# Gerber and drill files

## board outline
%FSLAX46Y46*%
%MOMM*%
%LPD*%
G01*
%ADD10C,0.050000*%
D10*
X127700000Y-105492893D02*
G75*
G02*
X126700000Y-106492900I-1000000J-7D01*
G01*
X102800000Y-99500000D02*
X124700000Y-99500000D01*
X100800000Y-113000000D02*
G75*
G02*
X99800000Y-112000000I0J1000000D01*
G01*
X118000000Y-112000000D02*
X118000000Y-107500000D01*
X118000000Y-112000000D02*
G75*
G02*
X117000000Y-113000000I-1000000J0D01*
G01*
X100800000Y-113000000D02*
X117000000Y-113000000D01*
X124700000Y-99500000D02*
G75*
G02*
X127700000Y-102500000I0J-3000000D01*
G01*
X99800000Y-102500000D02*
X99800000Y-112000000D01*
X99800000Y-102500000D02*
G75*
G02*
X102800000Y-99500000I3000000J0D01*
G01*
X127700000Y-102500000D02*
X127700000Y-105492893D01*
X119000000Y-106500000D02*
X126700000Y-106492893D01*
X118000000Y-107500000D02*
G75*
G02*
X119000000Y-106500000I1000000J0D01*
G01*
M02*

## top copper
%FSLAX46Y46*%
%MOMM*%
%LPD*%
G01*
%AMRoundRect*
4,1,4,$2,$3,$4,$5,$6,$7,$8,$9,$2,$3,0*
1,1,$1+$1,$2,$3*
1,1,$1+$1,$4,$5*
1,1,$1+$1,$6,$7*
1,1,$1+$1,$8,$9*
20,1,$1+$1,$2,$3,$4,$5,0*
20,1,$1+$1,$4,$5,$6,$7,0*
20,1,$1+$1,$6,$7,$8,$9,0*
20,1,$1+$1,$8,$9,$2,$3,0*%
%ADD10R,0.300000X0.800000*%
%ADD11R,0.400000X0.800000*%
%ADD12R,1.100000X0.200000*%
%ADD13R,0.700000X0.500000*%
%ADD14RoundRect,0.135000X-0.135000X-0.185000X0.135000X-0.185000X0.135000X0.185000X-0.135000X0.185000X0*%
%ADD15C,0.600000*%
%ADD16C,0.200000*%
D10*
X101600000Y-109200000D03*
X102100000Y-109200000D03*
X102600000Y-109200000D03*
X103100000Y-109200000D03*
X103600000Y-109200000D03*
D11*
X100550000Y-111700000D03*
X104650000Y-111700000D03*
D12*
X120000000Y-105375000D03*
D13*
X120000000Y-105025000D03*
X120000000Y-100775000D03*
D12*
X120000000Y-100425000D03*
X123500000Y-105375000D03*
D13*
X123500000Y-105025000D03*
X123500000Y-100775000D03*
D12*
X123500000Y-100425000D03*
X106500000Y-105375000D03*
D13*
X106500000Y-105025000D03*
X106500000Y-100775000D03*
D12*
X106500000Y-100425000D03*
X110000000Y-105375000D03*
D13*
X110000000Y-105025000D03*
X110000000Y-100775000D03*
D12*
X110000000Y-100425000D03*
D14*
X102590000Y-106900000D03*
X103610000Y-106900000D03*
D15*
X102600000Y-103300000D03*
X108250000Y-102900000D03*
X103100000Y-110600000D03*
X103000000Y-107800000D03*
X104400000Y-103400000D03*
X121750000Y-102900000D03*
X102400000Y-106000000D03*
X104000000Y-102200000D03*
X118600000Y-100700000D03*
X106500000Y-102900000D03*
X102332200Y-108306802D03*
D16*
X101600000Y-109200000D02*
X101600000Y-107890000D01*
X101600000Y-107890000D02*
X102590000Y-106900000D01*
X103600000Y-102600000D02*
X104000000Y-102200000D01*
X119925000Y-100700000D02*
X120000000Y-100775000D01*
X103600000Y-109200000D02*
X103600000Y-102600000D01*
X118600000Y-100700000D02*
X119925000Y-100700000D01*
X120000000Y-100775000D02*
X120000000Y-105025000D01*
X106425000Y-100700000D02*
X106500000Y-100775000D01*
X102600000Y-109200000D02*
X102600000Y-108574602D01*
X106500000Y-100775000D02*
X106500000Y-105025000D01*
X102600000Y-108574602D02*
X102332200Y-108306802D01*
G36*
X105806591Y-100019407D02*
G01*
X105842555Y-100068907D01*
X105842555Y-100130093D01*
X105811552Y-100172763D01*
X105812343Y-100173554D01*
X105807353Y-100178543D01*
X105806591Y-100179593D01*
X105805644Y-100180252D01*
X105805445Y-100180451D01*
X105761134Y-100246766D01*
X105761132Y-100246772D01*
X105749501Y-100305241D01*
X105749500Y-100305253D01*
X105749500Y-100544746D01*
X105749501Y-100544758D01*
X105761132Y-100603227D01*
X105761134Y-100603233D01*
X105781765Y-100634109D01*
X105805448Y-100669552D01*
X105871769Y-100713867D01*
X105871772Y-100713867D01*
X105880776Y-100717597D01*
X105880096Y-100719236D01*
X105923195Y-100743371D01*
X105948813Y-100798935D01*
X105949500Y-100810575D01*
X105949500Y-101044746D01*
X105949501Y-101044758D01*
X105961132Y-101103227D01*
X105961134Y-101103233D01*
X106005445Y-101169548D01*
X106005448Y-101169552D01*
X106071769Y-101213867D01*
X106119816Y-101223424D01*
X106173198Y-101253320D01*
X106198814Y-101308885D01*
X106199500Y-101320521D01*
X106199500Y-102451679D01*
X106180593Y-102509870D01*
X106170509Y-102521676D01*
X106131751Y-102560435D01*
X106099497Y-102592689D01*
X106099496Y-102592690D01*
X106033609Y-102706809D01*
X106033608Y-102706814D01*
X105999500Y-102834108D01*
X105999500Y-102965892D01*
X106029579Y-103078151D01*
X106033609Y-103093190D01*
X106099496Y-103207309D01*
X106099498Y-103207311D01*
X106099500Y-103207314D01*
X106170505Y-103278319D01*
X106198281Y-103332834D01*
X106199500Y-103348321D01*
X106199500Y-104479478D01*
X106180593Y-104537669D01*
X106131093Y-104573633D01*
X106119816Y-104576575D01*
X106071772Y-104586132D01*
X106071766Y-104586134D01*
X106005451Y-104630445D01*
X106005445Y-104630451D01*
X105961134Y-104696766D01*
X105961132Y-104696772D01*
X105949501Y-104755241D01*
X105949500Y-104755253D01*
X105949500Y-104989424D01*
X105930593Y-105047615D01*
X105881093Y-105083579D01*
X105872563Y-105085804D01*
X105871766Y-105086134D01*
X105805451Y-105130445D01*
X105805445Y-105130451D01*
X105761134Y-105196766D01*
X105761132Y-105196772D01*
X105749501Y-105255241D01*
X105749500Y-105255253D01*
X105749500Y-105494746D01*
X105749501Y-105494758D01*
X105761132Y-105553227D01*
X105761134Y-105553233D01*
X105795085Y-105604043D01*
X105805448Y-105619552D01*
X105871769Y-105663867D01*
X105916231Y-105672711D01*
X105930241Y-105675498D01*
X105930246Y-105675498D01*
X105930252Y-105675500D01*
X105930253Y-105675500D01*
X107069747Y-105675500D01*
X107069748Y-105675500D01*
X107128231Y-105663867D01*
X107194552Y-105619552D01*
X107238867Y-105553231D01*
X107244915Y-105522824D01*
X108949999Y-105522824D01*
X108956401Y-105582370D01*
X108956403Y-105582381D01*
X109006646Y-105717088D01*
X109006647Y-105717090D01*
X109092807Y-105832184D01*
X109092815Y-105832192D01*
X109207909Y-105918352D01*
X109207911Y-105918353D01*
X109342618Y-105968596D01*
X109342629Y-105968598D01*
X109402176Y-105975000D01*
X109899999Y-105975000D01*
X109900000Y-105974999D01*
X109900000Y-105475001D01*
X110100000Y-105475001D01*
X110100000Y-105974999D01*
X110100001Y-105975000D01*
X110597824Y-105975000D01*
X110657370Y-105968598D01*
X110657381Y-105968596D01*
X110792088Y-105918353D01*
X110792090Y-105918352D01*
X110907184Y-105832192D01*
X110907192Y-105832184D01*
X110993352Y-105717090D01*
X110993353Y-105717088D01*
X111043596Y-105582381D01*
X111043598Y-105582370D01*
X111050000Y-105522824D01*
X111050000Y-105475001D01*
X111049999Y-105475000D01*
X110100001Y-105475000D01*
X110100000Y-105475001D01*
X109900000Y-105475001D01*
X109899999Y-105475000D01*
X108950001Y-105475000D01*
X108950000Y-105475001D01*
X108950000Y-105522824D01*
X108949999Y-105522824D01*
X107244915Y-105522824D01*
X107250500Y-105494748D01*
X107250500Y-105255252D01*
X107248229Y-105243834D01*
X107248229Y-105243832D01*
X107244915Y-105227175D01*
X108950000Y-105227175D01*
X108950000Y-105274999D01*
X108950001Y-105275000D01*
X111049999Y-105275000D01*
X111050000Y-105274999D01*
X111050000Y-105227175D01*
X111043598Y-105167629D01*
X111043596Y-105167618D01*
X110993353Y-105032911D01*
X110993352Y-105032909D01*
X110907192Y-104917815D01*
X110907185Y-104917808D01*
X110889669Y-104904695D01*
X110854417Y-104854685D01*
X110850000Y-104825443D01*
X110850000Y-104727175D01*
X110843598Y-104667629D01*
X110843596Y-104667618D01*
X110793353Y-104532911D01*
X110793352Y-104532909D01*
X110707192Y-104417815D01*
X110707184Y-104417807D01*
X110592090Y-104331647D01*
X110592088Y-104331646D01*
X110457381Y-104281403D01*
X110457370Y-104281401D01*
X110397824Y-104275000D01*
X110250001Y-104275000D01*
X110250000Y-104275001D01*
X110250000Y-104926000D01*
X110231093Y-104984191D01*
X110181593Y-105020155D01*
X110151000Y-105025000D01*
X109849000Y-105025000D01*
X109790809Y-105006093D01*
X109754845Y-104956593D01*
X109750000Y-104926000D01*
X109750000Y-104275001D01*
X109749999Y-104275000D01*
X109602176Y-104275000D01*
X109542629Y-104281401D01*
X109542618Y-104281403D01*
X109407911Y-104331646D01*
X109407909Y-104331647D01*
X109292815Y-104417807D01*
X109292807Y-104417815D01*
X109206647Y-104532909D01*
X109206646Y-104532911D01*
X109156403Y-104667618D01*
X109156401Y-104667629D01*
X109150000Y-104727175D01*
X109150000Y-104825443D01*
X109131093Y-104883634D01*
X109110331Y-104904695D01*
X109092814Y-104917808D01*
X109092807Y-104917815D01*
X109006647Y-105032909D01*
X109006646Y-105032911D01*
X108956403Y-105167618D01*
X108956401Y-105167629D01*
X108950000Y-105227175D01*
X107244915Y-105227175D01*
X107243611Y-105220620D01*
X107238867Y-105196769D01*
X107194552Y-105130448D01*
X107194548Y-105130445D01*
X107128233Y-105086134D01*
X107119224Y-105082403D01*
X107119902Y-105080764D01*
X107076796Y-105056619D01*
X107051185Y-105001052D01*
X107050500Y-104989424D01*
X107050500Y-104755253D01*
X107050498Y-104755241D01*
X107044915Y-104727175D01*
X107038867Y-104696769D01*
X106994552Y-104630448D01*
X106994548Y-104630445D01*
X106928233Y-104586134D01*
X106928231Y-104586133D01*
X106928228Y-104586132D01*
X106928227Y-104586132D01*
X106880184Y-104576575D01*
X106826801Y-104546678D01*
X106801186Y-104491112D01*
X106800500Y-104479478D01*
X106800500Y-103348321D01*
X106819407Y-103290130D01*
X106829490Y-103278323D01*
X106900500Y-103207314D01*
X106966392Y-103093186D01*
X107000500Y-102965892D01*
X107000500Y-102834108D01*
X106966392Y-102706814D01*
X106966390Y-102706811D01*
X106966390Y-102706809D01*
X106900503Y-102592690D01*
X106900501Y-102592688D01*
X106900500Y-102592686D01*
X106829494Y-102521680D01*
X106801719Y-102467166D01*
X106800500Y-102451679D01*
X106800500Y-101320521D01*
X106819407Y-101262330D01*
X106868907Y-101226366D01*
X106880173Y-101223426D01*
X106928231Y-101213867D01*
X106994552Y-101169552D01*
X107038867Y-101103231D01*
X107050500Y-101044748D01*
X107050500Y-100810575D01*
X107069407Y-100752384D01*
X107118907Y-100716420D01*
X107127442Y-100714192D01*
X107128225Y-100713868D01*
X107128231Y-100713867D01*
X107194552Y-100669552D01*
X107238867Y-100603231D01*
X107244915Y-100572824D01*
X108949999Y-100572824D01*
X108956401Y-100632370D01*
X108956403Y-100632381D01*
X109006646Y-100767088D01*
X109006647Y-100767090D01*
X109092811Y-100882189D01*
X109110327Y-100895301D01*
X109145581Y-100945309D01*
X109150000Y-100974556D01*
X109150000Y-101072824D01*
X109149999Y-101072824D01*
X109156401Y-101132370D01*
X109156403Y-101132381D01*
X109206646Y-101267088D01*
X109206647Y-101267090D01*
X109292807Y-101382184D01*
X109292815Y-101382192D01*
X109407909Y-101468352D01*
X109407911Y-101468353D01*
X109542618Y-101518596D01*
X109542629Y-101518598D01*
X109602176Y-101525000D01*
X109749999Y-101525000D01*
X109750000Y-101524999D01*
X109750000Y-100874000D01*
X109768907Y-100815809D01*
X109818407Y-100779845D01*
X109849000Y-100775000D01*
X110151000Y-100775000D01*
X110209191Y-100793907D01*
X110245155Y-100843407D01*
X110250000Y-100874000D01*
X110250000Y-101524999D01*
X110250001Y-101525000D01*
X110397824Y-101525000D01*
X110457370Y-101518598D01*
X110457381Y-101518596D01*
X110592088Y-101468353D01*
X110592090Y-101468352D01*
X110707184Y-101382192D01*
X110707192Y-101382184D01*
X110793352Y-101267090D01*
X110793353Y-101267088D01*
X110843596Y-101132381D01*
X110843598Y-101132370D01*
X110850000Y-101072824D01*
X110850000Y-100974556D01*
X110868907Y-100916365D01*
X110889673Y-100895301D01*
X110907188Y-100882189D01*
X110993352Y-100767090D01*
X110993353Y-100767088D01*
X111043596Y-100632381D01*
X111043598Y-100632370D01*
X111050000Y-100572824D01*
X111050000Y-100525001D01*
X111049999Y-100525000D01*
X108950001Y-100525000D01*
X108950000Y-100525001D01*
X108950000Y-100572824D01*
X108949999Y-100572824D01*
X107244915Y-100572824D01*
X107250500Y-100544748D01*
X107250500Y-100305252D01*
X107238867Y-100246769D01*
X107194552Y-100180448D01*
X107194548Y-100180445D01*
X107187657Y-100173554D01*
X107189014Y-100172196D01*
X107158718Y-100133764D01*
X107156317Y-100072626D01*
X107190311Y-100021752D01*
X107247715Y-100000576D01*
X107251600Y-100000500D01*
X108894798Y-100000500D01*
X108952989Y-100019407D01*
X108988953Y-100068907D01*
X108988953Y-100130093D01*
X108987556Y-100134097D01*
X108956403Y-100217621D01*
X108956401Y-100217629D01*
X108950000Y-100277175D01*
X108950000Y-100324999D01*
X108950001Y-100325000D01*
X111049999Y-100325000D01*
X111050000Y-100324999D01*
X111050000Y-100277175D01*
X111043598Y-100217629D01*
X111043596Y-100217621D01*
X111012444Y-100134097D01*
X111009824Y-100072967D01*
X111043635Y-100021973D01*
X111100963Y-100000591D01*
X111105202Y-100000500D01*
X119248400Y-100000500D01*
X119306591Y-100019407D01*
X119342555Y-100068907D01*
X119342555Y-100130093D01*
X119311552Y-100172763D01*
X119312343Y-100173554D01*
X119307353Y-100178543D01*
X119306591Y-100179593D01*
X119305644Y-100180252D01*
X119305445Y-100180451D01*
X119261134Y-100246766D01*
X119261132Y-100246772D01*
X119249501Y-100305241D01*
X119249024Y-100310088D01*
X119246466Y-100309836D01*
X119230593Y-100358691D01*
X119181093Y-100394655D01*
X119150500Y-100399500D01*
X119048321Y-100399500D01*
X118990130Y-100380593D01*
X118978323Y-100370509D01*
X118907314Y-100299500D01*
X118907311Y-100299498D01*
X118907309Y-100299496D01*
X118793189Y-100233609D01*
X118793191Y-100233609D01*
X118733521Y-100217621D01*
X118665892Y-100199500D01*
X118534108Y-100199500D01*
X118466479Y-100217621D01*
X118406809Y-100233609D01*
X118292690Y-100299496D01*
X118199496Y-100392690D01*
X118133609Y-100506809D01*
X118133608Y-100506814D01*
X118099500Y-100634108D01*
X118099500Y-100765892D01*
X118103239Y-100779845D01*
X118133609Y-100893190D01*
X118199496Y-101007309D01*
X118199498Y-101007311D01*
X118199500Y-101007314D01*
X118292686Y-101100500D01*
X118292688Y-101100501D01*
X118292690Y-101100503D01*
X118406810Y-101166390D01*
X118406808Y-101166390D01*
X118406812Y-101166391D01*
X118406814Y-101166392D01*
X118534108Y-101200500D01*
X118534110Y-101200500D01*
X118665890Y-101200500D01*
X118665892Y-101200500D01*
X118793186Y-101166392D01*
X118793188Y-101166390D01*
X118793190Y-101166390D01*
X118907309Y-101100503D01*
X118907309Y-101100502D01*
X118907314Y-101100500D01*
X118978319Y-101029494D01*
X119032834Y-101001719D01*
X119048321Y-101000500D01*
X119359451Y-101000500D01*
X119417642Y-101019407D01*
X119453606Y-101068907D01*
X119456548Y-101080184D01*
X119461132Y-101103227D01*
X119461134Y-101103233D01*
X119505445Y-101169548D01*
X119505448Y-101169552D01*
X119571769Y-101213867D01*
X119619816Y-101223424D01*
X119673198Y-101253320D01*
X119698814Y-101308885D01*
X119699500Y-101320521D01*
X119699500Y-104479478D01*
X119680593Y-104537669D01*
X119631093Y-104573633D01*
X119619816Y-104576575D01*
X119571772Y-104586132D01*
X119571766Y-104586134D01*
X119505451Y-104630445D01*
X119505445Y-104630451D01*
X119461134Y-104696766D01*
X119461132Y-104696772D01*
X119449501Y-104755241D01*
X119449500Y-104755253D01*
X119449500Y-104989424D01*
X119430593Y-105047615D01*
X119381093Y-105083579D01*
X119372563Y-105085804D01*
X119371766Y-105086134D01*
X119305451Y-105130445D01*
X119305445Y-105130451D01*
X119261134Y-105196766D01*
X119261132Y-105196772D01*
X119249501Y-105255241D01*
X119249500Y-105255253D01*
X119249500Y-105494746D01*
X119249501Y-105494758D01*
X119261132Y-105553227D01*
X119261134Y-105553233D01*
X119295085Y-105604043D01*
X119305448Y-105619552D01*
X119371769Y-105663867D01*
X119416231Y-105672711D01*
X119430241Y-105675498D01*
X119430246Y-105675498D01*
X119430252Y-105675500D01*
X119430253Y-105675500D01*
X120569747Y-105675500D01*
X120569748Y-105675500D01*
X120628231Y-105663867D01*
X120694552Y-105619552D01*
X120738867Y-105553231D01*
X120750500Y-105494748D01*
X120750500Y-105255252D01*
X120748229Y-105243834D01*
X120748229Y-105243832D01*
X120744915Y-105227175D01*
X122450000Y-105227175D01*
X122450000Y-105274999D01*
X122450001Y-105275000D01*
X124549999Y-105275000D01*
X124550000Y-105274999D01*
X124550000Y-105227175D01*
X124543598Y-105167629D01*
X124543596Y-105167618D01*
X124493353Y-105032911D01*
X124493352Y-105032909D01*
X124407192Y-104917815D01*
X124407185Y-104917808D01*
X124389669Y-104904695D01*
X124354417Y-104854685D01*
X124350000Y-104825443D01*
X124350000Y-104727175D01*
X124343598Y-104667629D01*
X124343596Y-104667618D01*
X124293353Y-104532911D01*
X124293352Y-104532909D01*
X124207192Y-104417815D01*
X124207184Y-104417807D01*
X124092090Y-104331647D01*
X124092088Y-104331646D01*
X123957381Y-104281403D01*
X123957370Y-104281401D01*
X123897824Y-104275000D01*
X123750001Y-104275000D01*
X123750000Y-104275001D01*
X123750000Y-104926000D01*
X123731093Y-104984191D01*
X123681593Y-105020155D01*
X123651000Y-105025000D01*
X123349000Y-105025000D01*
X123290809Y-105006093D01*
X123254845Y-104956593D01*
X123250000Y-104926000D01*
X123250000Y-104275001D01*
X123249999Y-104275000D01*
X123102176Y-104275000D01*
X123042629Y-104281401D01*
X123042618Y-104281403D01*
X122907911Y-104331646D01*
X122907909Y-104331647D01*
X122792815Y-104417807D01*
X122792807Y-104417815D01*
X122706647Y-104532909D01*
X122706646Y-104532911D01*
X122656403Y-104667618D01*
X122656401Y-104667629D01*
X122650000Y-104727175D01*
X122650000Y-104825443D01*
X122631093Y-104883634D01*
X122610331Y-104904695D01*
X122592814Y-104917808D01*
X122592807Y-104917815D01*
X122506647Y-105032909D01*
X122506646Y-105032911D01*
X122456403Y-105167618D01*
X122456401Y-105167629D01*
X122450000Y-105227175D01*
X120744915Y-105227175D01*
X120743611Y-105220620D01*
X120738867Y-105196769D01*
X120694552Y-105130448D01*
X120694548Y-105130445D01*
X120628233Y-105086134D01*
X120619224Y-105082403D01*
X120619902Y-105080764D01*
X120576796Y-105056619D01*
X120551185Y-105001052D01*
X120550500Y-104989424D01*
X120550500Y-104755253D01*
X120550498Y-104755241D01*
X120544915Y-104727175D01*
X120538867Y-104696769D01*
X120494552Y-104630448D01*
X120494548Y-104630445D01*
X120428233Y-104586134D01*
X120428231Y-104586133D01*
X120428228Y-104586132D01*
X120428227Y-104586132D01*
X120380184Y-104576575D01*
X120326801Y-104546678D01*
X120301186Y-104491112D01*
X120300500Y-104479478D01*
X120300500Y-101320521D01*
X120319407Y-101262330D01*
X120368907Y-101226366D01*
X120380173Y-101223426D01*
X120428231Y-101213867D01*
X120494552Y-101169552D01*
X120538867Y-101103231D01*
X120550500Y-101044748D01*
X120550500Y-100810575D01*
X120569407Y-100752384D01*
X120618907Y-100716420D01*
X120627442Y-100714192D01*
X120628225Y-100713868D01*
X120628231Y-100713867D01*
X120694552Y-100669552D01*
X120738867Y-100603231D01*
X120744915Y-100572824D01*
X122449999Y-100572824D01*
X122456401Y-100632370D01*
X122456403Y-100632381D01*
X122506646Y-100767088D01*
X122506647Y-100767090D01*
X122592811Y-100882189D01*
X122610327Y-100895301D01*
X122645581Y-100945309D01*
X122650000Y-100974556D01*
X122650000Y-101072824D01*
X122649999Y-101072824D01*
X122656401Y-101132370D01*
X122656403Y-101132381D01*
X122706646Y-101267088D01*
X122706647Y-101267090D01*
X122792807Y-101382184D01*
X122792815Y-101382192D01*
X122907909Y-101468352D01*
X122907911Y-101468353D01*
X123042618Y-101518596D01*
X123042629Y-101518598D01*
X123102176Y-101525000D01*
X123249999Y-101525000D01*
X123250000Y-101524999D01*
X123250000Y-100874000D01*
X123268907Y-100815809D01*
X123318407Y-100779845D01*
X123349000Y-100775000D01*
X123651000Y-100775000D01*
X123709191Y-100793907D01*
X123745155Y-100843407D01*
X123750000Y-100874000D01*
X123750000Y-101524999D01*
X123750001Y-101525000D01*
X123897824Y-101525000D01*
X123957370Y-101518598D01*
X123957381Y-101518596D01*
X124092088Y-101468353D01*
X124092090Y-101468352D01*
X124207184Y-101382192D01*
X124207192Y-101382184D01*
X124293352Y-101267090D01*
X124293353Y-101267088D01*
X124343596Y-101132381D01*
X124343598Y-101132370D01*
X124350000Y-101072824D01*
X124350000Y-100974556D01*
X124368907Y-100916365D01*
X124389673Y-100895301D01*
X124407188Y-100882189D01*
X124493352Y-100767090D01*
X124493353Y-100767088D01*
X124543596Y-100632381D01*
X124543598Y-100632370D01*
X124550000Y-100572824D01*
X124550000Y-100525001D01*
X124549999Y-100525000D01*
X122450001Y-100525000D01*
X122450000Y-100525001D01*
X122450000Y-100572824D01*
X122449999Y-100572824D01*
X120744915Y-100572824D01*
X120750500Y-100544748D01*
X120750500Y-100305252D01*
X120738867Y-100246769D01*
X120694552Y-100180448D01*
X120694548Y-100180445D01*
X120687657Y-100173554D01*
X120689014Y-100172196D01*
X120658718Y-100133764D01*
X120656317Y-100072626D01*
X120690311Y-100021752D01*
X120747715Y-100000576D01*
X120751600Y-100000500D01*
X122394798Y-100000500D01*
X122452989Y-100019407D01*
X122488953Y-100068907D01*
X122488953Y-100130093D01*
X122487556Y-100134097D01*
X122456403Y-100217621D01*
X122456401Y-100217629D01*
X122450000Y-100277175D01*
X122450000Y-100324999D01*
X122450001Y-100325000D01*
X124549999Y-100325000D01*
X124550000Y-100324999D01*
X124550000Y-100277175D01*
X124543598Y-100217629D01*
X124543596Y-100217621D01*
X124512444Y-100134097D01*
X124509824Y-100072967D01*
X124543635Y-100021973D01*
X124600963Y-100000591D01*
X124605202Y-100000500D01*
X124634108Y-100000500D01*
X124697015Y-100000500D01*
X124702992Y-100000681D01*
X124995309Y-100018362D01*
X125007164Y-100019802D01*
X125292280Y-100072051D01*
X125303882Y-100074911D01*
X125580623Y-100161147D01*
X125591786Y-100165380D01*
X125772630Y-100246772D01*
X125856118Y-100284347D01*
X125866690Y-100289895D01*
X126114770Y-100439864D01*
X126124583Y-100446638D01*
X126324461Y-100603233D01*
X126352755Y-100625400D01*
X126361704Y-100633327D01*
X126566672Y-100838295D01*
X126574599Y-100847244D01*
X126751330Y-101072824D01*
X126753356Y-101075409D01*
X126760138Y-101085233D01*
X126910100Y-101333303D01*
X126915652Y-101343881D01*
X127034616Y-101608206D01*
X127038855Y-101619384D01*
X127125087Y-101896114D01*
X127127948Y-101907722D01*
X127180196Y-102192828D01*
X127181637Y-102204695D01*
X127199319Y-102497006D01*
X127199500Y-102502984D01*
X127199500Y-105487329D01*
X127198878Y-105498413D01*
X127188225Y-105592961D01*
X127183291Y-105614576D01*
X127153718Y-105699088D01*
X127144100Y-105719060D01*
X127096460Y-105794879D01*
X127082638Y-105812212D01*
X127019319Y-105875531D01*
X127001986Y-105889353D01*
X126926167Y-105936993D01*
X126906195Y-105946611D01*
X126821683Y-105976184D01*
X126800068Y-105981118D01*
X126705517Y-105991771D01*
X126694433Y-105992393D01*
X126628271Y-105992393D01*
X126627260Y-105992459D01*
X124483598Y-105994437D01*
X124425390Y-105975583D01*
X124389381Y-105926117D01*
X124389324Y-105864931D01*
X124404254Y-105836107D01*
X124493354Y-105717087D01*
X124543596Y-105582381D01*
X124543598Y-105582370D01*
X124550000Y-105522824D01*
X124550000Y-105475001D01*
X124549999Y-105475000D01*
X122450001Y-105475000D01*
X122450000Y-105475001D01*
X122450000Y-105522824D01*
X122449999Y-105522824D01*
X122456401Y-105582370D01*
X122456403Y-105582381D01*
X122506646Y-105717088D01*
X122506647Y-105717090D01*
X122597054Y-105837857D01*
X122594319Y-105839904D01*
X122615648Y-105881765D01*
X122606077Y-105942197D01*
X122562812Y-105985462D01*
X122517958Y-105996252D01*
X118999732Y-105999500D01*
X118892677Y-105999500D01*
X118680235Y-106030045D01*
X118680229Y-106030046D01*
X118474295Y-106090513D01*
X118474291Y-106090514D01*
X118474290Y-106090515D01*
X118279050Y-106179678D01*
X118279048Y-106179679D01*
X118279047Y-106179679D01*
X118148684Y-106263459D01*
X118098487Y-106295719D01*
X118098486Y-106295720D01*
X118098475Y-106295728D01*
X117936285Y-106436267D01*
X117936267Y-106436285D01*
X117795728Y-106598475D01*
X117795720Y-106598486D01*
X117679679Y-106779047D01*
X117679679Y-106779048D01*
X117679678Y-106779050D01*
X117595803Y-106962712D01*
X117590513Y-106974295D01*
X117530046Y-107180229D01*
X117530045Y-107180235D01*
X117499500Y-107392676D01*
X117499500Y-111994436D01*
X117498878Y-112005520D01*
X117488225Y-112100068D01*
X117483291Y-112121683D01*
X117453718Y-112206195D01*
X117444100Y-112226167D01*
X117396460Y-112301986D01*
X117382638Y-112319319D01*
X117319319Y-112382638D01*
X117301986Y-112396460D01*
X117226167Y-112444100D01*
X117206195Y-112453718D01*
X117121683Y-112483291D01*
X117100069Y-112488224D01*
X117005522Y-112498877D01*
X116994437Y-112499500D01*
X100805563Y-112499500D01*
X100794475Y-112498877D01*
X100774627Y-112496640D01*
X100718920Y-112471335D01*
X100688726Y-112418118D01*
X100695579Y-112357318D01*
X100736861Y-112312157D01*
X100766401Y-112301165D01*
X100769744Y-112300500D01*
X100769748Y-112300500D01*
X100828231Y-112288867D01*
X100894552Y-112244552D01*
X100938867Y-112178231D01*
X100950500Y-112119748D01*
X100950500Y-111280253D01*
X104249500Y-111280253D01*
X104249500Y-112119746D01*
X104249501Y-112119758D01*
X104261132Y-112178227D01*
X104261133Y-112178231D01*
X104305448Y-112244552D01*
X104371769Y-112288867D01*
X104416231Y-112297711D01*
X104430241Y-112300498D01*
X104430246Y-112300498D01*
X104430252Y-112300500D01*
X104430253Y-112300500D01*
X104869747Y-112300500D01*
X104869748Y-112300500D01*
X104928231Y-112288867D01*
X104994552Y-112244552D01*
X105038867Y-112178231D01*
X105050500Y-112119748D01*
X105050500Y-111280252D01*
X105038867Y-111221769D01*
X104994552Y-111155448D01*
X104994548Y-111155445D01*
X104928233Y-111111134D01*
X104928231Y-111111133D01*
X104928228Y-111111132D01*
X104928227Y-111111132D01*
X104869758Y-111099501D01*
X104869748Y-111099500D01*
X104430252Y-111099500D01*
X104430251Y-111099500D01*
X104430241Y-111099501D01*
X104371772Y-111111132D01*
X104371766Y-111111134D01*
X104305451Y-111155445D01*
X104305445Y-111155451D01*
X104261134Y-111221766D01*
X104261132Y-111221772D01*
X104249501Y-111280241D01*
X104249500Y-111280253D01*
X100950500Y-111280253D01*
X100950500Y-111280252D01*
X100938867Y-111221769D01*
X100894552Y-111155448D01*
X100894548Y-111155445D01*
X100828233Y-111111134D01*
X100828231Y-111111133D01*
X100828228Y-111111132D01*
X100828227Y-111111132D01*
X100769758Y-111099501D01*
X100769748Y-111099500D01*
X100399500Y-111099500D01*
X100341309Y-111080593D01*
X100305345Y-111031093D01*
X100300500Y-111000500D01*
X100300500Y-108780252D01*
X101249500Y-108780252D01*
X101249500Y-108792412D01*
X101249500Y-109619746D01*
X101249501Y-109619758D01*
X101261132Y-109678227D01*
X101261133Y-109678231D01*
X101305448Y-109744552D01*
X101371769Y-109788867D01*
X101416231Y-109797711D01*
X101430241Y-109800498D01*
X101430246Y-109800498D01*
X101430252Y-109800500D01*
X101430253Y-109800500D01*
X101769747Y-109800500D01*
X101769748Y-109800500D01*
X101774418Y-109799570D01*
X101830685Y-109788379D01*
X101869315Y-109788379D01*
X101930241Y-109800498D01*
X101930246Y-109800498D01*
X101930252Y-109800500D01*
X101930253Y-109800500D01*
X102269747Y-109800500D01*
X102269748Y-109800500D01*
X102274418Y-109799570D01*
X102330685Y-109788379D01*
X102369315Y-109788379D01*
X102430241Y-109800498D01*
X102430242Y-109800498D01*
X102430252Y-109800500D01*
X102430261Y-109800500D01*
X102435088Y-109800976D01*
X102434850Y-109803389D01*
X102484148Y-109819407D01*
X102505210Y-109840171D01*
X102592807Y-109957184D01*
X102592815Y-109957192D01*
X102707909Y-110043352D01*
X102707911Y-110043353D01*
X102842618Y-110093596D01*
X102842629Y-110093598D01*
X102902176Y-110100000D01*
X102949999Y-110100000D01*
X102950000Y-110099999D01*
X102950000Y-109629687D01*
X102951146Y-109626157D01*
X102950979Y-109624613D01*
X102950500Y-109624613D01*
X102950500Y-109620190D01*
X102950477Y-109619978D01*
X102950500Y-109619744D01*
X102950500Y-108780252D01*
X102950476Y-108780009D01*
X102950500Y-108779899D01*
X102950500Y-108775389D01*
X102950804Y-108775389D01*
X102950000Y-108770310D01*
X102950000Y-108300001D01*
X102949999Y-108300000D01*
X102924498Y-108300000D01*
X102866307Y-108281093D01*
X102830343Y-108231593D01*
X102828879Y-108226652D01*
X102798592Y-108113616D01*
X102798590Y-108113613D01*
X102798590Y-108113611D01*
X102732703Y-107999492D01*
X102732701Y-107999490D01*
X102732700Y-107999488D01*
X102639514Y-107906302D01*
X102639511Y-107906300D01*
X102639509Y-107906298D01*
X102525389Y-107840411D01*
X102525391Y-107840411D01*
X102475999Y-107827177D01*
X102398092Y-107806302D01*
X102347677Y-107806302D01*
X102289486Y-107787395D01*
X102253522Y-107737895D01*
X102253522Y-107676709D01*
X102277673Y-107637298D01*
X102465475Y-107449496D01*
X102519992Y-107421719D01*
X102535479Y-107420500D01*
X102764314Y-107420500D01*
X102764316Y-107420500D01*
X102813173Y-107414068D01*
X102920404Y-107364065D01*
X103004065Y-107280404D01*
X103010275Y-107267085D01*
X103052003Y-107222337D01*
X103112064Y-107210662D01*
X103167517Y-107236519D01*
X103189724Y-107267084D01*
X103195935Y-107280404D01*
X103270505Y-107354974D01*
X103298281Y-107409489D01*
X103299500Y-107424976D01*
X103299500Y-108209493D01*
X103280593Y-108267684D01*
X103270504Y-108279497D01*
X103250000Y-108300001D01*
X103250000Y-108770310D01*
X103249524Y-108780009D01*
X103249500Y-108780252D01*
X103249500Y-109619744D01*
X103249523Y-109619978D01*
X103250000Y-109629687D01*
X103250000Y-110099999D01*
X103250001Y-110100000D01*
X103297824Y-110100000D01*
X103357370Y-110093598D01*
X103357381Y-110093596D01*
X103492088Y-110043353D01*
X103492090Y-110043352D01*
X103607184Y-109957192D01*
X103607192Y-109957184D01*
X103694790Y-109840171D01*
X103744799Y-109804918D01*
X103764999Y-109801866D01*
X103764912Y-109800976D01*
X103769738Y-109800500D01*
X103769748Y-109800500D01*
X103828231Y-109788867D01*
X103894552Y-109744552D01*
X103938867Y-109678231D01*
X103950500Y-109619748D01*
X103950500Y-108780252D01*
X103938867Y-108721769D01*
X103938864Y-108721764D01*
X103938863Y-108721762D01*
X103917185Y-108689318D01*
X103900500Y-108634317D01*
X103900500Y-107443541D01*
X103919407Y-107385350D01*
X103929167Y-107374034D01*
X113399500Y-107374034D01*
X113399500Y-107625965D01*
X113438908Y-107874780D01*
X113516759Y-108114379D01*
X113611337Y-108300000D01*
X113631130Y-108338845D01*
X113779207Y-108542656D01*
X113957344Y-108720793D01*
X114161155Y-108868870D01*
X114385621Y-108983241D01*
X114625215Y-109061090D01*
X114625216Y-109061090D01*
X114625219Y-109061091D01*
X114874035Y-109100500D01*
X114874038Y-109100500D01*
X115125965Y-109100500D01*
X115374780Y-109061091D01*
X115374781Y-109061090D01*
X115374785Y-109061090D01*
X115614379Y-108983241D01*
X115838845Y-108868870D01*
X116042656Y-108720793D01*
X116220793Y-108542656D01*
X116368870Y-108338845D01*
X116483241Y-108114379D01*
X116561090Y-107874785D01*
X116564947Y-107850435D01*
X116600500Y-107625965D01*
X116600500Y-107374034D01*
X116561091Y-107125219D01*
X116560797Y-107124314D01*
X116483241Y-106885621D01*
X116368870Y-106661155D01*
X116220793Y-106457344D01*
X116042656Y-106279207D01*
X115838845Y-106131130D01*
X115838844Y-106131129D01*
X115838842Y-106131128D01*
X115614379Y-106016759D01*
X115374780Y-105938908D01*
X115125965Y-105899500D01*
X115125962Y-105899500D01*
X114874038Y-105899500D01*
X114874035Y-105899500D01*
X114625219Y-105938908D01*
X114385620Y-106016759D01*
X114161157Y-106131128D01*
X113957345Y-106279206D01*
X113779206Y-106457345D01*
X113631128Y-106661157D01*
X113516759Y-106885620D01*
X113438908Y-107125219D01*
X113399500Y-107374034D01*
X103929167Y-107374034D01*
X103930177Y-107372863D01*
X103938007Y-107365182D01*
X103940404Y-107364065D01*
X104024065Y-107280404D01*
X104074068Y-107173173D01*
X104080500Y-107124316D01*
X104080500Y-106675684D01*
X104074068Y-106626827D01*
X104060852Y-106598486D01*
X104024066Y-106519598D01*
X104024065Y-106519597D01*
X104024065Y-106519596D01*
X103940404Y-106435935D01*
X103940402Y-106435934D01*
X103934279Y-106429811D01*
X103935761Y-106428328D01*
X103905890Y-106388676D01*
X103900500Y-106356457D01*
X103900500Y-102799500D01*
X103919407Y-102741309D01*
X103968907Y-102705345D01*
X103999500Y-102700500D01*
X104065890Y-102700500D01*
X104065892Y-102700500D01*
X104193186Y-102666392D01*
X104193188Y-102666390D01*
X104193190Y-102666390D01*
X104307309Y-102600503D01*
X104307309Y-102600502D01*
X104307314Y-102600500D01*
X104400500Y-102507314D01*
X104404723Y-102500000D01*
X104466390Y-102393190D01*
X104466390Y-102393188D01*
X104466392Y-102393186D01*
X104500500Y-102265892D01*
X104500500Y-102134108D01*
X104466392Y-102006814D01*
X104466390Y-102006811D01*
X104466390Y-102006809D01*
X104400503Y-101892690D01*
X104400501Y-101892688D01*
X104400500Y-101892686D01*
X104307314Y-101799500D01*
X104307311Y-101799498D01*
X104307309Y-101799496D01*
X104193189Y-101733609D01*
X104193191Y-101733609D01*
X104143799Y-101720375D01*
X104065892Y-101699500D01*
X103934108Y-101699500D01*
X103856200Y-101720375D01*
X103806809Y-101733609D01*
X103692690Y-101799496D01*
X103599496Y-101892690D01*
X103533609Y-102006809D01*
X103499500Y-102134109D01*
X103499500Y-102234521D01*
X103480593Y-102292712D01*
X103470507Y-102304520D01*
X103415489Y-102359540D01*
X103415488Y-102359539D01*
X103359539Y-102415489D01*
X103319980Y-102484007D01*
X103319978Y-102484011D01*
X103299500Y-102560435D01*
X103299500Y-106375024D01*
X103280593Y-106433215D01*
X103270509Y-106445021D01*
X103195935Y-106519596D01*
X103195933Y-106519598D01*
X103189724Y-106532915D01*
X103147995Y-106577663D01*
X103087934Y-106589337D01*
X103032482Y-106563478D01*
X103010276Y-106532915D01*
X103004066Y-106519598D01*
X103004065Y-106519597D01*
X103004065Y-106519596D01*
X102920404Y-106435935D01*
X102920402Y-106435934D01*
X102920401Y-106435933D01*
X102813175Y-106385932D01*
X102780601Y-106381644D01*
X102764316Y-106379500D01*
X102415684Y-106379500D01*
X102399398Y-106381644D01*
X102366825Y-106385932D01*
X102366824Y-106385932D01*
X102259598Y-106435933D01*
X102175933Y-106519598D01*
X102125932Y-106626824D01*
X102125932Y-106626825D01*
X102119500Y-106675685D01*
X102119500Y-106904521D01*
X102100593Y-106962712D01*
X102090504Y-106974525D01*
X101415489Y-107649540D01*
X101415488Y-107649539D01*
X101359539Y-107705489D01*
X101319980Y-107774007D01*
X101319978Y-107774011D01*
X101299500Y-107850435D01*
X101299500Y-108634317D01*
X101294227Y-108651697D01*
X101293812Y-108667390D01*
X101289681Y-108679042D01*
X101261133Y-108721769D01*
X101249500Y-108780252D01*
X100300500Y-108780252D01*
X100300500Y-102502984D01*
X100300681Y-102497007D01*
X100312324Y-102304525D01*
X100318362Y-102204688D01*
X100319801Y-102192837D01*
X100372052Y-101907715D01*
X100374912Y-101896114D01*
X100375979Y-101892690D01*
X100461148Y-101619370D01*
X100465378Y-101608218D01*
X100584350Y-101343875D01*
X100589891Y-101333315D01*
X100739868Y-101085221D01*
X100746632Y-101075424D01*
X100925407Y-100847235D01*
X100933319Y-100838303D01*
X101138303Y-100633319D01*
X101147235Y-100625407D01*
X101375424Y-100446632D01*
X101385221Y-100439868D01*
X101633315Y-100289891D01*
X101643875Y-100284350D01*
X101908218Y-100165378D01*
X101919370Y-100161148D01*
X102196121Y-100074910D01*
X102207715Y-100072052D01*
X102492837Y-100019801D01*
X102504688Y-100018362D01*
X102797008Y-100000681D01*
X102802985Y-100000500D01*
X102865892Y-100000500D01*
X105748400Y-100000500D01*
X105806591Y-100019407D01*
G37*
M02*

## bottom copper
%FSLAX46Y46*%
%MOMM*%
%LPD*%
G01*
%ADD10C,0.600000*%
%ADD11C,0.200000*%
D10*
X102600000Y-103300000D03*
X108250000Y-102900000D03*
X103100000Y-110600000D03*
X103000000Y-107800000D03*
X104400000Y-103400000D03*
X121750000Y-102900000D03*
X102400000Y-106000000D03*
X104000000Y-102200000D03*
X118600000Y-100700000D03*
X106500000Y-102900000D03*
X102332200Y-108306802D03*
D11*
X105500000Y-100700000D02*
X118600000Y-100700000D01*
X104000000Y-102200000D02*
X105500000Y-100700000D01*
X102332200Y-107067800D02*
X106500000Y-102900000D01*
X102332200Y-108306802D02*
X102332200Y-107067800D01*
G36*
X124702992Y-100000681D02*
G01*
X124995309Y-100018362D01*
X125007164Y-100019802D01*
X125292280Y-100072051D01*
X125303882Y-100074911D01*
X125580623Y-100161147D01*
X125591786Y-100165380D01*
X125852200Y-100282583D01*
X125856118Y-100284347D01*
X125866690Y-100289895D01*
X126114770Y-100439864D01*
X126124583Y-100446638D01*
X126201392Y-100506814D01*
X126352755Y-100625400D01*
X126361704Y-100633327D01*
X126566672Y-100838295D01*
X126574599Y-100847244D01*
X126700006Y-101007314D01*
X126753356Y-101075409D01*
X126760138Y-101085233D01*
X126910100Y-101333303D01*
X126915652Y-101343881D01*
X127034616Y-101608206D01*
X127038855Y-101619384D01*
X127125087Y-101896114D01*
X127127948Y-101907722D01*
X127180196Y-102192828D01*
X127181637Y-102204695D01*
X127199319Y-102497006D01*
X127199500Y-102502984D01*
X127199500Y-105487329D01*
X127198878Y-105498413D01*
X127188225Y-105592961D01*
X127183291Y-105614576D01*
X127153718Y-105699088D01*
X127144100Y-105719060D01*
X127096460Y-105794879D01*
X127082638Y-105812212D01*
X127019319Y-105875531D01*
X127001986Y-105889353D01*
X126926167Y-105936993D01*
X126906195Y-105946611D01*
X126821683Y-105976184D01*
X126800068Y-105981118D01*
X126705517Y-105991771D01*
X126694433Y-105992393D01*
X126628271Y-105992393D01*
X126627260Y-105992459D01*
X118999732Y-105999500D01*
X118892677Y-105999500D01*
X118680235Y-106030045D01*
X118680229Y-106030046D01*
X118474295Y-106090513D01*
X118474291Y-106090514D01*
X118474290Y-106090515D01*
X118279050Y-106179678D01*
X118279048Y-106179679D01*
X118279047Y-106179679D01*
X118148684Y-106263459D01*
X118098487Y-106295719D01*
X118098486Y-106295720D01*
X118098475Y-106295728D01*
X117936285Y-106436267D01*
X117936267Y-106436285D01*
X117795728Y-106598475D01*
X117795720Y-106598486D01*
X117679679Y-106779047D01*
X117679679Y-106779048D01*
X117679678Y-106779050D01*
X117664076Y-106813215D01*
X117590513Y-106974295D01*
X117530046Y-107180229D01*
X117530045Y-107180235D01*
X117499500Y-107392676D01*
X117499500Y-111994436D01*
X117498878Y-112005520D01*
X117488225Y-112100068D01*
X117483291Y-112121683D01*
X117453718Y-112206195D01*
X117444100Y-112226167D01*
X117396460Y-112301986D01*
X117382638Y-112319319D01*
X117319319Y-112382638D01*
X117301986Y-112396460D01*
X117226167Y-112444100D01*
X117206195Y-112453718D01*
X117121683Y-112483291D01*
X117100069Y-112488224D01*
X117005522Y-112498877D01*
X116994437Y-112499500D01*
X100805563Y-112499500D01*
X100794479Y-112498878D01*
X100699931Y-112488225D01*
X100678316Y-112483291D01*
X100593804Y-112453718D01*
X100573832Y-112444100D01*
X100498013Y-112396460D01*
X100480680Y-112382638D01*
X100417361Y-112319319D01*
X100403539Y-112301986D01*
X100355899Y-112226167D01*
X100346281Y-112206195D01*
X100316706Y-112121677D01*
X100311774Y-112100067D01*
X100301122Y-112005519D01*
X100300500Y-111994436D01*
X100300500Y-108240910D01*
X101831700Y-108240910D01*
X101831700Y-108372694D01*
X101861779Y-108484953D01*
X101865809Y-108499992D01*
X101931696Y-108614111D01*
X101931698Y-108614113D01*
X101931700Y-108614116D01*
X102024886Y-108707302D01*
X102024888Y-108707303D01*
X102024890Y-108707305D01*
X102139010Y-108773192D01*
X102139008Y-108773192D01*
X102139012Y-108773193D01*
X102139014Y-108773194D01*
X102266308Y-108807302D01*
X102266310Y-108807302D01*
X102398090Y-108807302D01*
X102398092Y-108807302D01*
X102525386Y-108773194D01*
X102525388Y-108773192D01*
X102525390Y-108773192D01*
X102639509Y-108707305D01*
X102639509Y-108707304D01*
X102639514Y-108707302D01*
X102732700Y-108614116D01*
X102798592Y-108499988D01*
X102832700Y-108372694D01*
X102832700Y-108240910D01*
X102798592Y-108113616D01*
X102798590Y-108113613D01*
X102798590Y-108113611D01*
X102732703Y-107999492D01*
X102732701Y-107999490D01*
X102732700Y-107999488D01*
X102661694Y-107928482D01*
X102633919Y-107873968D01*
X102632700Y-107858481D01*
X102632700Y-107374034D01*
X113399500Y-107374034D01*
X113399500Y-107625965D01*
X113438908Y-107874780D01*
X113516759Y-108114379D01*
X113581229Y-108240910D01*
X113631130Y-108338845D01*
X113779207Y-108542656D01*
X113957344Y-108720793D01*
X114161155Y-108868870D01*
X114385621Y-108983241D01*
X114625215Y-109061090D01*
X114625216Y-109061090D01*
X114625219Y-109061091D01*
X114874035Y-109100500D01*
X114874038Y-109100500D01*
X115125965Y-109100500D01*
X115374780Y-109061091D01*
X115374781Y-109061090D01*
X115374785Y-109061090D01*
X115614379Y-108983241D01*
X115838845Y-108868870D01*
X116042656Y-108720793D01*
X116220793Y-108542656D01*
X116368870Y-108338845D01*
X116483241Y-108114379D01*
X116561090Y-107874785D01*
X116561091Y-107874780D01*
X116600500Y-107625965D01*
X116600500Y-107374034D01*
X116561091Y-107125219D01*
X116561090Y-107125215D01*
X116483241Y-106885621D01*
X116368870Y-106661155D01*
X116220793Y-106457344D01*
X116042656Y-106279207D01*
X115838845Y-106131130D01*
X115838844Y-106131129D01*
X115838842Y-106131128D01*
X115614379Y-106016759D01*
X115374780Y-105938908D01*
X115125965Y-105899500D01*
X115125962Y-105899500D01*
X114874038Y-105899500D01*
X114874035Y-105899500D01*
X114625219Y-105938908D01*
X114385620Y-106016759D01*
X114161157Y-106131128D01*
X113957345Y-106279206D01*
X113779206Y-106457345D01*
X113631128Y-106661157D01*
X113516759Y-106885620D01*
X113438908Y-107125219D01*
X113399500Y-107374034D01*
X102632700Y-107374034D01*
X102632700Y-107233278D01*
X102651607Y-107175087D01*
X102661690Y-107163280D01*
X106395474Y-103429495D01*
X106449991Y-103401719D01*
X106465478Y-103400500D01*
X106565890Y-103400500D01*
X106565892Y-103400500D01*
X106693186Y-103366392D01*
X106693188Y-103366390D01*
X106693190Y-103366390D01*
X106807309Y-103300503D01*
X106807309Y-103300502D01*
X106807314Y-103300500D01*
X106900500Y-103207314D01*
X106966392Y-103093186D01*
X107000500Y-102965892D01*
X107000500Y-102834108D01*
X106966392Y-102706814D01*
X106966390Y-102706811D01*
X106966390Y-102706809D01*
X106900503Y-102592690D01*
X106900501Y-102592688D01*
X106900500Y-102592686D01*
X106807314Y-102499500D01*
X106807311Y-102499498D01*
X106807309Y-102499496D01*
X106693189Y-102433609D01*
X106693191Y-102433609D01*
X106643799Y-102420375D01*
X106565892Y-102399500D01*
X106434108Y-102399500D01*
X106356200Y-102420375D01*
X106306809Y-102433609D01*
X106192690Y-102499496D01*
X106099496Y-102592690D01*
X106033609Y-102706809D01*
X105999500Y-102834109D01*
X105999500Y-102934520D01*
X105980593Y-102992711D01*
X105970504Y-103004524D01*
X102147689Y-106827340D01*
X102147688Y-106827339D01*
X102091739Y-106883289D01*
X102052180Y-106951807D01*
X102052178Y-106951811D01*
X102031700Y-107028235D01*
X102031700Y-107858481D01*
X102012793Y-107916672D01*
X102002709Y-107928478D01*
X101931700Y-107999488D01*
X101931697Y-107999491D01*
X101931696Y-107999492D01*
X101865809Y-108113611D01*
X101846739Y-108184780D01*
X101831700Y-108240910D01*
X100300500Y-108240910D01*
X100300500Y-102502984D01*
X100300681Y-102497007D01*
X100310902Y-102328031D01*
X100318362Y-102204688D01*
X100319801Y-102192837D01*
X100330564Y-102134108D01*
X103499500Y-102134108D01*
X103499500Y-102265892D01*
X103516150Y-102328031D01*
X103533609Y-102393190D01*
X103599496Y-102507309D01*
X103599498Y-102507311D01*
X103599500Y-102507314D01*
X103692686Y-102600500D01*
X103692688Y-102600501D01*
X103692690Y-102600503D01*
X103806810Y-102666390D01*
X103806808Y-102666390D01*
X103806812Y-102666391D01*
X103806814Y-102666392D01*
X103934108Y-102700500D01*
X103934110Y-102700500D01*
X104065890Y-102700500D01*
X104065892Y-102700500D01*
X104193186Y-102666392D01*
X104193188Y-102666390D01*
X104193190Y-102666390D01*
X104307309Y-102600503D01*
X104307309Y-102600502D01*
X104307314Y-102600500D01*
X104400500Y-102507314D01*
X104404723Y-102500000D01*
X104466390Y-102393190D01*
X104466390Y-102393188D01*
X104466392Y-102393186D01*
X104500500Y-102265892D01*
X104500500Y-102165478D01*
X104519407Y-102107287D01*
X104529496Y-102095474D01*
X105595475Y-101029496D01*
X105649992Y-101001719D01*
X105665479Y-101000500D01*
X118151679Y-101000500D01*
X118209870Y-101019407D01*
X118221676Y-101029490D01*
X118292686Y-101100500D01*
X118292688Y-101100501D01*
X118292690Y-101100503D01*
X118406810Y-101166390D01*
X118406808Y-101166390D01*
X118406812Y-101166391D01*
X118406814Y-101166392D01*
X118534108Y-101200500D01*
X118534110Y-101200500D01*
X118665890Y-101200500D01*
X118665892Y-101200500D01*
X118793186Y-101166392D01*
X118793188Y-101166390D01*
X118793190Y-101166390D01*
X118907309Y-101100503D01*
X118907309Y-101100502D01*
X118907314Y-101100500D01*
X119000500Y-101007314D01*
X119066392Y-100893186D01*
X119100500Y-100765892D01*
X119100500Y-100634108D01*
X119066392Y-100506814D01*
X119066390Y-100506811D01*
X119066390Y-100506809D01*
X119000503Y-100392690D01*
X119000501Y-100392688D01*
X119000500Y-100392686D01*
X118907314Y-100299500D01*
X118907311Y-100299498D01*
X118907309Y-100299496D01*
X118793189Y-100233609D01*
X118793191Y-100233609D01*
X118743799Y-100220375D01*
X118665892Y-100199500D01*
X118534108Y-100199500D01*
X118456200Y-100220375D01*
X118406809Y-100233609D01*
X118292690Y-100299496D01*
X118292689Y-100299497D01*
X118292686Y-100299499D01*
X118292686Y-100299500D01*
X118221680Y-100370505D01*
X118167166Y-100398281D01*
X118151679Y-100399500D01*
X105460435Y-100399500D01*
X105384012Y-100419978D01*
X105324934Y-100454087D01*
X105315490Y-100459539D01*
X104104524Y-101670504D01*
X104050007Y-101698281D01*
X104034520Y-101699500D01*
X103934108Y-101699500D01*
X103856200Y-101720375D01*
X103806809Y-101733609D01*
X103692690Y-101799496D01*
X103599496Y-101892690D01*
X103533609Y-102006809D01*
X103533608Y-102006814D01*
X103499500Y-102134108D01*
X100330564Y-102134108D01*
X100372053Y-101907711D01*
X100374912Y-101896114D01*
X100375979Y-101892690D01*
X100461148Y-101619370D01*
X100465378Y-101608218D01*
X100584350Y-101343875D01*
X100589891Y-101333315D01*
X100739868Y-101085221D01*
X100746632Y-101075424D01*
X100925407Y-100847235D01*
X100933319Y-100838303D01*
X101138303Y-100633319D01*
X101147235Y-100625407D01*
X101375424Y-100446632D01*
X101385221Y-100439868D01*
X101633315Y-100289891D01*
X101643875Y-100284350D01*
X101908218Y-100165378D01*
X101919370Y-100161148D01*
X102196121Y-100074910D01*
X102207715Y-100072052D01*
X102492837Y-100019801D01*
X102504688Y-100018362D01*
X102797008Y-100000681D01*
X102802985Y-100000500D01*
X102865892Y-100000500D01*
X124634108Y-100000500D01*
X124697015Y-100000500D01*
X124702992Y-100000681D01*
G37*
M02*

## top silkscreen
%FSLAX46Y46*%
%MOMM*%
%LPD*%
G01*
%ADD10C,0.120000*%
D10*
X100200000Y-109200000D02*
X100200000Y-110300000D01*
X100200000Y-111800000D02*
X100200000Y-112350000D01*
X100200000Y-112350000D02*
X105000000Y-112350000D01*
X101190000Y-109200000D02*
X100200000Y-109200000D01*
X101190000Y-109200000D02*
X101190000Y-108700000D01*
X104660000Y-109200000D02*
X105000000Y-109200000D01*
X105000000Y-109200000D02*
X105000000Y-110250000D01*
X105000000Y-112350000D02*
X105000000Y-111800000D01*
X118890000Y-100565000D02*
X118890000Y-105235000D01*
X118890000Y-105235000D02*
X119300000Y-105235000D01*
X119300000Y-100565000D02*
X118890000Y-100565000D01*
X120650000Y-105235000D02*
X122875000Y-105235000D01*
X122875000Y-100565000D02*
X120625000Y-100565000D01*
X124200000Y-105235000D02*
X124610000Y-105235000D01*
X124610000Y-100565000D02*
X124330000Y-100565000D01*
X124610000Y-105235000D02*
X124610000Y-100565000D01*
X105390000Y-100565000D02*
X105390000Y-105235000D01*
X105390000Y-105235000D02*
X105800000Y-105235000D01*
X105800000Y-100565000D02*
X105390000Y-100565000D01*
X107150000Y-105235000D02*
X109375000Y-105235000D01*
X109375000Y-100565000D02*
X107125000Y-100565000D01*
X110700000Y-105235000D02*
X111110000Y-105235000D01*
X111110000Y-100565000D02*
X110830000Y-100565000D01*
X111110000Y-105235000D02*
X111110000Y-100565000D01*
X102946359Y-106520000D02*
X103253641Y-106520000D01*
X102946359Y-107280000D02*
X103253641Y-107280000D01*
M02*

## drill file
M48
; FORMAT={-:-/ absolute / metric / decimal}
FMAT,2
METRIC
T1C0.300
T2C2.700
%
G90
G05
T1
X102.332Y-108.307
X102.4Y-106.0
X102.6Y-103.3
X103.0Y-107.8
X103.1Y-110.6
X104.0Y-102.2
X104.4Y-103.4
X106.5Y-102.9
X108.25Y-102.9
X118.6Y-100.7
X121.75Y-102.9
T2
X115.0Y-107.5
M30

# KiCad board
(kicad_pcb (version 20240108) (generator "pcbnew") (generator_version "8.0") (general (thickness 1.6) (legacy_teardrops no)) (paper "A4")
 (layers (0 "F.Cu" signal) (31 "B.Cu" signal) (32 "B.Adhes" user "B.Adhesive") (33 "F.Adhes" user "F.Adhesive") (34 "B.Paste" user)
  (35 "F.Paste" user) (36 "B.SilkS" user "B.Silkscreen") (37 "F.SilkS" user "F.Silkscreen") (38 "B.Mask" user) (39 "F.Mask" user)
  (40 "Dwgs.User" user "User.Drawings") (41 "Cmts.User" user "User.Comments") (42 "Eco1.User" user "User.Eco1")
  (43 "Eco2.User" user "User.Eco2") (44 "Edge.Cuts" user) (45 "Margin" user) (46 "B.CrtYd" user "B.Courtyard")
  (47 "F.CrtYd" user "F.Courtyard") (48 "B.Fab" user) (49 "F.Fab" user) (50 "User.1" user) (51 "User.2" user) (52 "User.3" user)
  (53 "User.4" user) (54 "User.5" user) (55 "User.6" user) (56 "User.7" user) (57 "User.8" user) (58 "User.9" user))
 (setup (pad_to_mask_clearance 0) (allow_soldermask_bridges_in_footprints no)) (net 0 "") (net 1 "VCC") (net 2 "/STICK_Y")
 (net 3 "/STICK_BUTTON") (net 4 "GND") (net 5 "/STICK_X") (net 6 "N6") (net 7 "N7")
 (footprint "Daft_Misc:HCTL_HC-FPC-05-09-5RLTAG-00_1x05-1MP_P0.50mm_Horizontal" (layer "F.Cu") (at 102.6 111)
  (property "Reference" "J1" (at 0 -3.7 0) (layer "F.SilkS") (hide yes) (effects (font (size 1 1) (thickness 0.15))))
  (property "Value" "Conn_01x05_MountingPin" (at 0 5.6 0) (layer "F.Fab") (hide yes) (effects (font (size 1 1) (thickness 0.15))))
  (fp_line (start -2.4 -1.8) (end -2.4 -0.7) (stroke (width 0.12) (type solid)) (layer "F.SilkS"))
  (fp_line (start -2.4 0.8) (end -2.4 1.35) (stroke (width 0.12) (type solid)) (layer "F.SilkS"))
  (fp_line (start -2.4 1.35) (end 2.4 1.35) (stroke (width 0.12) (type solid)) (layer "F.SilkS"))
  (fp_line (start -1.41 -1.8) (end -2.4 -1.8) (stroke (width 0.12) (type solid)) (layer "F.SilkS"))
  (fp_line (start -1.41 -1.8) (end -1.41 -2.3) (stroke (width 0.12) (type solid)) (layer "F.SilkS"))
  (fp_line (start 2.06 -1.8) (end 2.4 -1.8) (stroke (width 0.12) (type solid)) (layer "F.SilkS"))
  (fp_line (start 2.4 -1.8) (end 2.4 -0.75) (stroke (width 0.12) (type solid)) (layer "F.SilkS"))
  (fp_line (start 2.4 1.35) (end 2.4 0.8) (stroke (width 0.12) (type solid)) (layer "F.SilkS"))
  (pad "1" smd rect (at -1 -1.8) (size 0.3 0.8) (layers "F.Cu" "F.Paste" "F.Mask") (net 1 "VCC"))
  (pad "2" smd rect (at -0.5 -1.8) (size 0.3 0.8) (layers "F.Cu" "F.Paste" "F.Mask") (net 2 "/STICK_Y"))
  (pad "3" smd rect (at 0 -1.8) (size 0.3 0.8) (layers "F.Cu" "F.Paste" "F.Mask") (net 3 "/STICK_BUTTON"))
  (pad "4" smd rect (at 0.5 -1.8) (size 0.3 0.8) (layers "F.Cu" "F.Paste" "F.Mask") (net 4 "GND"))
  (pad "5" smd rect (at 1 -1.8) (size 0.3 0.8) (layers "F.Cu" "F.Paste" "F.Mask") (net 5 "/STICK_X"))
  (pad "MP" smd rect (at -2.05 0.7) (size 0.4 0.8) (layers "F.Cu" "F.Paste" "F.Mask") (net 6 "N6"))
  (pad "MP" smd rect (at 2.05 0.7) (size 0.4 0.8) (layers "F.Cu" "F.Paste" "F.Mask") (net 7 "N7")))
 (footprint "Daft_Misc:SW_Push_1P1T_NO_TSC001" (layer "F.Cu") (at 121.75 102.9 90)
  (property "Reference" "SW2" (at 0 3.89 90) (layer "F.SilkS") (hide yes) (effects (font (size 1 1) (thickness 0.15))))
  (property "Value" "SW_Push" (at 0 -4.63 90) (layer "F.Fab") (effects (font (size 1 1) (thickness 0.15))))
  (fp_line (start 2.335 -2.86) (end -2.335 -2.86) (stroke (width 0.12) (type solid)) (layer "F.SilkS"))
  (fp_line (start -2.335 -2.86) (end -2.335 -2.45) (stroke (width 0.12) (type solid)) (layer "F.SilkS"))
  (fp_line (start 2.335 -2.45) (end 2.335 -2.86) (stroke (width 0.12) (type solid)) (layer "F.SilkS"))
  (fp_line (start -2.335 -1.1) (end -2.335 1.125) (stroke (width 0.12) (type solid)) (layer "F.SilkS"))
  (fp_line (start 2.335 1.125) (end 2.335 -1.125) (stroke (width 0.12) (type solid)) (layer "F.SilkS"))
  (fp_line (start -2.335 2.45) (end -2.335 2.86) (stroke (width 0.12) (type solid)) (layer "F.SilkS"))
  (fp_line (start 2.335 2.86) (end 2.335 2.58) (stroke (width 0.12) (type solid)) (layer "F.SilkS"))
  (fp_line (start -2.335 2.86) (end 2.335 2.86) (stroke (width 0.12) (type solid)) (layer "F.SilkS"))
  (pad "1" smd rect (at -2.475 -1.75 90) (size 0.2 1.1) (layers "F.Cu" "F.Paste" "F.Mask") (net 5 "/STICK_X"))
  (pad "1" smd rect (at -2.125 -1.75 90) (size 0.5 0.7) (layers "F.Cu" "F.Paste" "F.Mask") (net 5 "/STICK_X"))
  (pad "1" smd rect (at 2.125 -1.75 90) (size 0.5 0.7) (layers "F.Cu" "F.Paste" "F.Mask") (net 5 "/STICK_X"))
  (pad "1" smd rect (at 2.475 -1.75 90) (size 0.2 1.1) (layers "F.Cu" "F.Paste" "F.Mask") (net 5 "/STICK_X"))
  (pad "2" smd rect (at -2.475 1.75 90) (size 0.2 1.1) (layers "F.Cu" "F.Paste" "F.Mask") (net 4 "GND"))
  (pad "2" smd rect (at -2.125 1.75 90) (size 0.5 0.7) (layers "F.Cu" "F.Paste" "F.Mask") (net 4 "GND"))
  (pad "2" smd rect (at 2.125 1.75 90) (size 0.5 0.7) (layers "F.Cu" "F.Paste" "F.Mask") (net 4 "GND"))
  (pad "2" smd rect (at 2.475 1.75 90) (size 0.2 1.1) (layers "F.Cu" "F.Paste" "F.Mask") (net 4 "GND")))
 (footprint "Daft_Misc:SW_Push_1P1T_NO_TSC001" (layer "F.Cu") (at 108.25 102.9 90)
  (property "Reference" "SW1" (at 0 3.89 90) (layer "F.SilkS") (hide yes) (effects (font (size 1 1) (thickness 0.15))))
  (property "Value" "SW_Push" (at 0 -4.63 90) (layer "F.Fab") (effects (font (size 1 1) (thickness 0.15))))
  (fp_line (start 2.335 -2.86) (end -2.335 -2.86) (stroke (width 0.12) (type solid)) (layer "F.SilkS"))
  (fp_line (start -2.335 -2.86) (end -2.335 -2.45) (stroke (width 0.12) (type solid)) (layer "F.SilkS"))
  (fp_line (start 2.335 -2.45) (end 2.335 -2.86) (stroke (width 0.12) (type solid)) (layer "F.SilkS"))
  (fp_line (start -2.335 -1.1) (end -2.335 1.125) (stroke (width 0.12) (type solid)) (layer "F.SilkS"))
  (fp_line (start 2.335 1.125) (end 2.335 -1.125) (stroke (width 0.12) (type solid)) (layer "F.SilkS"))
  (fp_line (start -2.335 2.45) (end -2.335 2.86) (stroke (width 0.12) (type solid)) (layer "F.SilkS"))
  (fp_line (start 2.335 2.86) (end 2.335 2.58) (stroke (width 0.12) (type solid)) (layer "F.SilkS"))
  (fp_line (start -2.335 2.86) (end 2.335 2.86) (stroke (width 0.12) (type solid)) (layer "F.SilkS"))
  (pad "1" smd rect (at -2.475 -1.75 90) (size 0.2 1.1) (layers "F.Cu" "F.Paste" "F.Mask") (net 3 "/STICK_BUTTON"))
  (pad "1" smd rect (at -2.125 -1.75 90) (size 0.5 0.7) (layers "F.Cu" "F.Paste" "F.Mask") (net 3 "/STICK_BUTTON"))
  (pad "1" smd rect (at 2.125 -1.75 90) (size 0.5 0.7) (layers "F.Cu" "F.Paste" "F.Mask") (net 3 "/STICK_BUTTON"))
  (pad "1" smd rect (at 2.475 -1.75 90) (size 0.2 1.1) (layers "F.Cu" "F.Paste" "F.Mask") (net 3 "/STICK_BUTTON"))
  (pad "2" smd rect (at -2.475 1.75 90) (size 0.2 1.1) (layers "F.Cu" "F.Paste" "F.Mask") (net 4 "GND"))
  (pad "2" smd rect (at -2.125 1.75 90) (size 0.5 0.7) (layers "F.Cu" "F.Paste" "F.Mask") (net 4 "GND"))
  (pad "2" smd rect (at 2.125 1.75 90) (size 0.5 0.7) (layers "F.Cu" "F.Paste" "F.Mask") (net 4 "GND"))
  (pad "2" smd rect (at 2.475 1.75 90) (size 0.2 1.1) (layers "F.Cu" "F.Paste" "F.Mask") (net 4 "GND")))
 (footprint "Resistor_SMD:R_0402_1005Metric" (layer "F.Cu") (at 103.1 106.9)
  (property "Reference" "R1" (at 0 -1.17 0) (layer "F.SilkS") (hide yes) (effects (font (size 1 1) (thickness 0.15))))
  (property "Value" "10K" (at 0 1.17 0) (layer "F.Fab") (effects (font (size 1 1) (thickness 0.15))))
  (fp_line (start -0.153641 -0.38) (end 0.153641 -0.38) (stroke (width 0.12) (type solid)) (layer "F.SilkS"))
  (fp_line (start -0.153641 0.38) (end 0.153641 0.38) (stroke (width 0.12) (type solid)) (layer "F.SilkS"))
  (pad "1" smd roundrect (at -0.51 0) (size 0.54 0.64) (layers "F.Cu" "F.Paste" "F.Mask") (roundrect_rratio 0.25) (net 1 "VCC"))
  (pad "2" smd roundrect (at 0.51 0) (size 0.54 0.64) (layers "F.Cu" "F.Paste" "F.Mask") (roundrect_rratio 0.25) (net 5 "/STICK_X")))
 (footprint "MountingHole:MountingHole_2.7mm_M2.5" (layer "F.Cu") (at 115 107.5)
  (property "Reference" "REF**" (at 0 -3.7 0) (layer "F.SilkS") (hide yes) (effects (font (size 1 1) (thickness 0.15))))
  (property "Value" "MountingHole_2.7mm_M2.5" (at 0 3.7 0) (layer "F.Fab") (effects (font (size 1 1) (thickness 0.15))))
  (pad "" np_thru_hole circle (at 0 0) (size 2.7 2.7) (drill 2.7) (layers "*.Cu" "*.Mask")))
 (gr_arc (start 127.7 105.492893) (mid 127.407107 106.2) (end 126.7 106.492893) (stroke (width 0.05) (type default)) (layer "Edge.Cuts"))
 (gr_line (start 102.8 99.5) (end 124.7 99.5) (stroke (width 0.05) (type default)) (layer "Edge.Cuts"))
 (gr_arc (start 100.8 113) (mid 100.092893 112.707107) (end 99.8 112) (stroke (width 0.05) (type default)) (layer "Edge.Cuts"))
 (gr_line (start 118 112) (end 118 107.5) (stroke (width 0.05) (type default)) (layer "Edge.Cuts"))
 (gr_arc (start 118 112) (mid 117.707107 112.707107) (end 117 113) (stroke (width 0.05) (type default)) (layer "Edge.Cuts"))
 (gr_line (start 100.8 113) (end 117 113) (stroke (width 0.05) (type default)) (layer "Edge.Cuts"))
 (gr_arc (start 124.7 99.5) (mid 126.82132 100.37868) (end 127.7 102.5) (stroke (width 0.05) (type default)) (layer "Edge.Cuts"))
 (gr_line (start 99.8 102.5) (end 99.8 112) (stroke (width 0.05) (type default)) (layer "Edge.Cuts"))
 (gr_arc (start 99.8 102.5) (mid 100.67868 100.37868) (end 102.8 99.5) (stroke (width 0.05) (type default)) (layer "Edge.Cuts"))
 (gr_line (start 127.7 102.5) (end 127.7 105.492893) (stroke (width 0.05) (type default)) (layer "Edge.Cuts"))
 (gr_line (start 119 106.5) (end 126.7 106.492893) (stroke (width 0.05) (type default)) (layer "Edge.Cuts"))
 (gr_arc (start 118 107.5) (mid 118.292893 106.792893) (end 119 106.5) (stroke (width 0.05) (type default)) (layer "Edge.Cuts"))
 (segment (start 101.6 109.2) (end 101.6 107.89) (width 0.2) (layer "F.Cu") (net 1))
 (segment (start 101.6 107.89) (end 102.59 106.9) (width 0.2) (layer "F.Cu") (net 1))
 (via (at 102.6 103.3) (size 0.6) (drill 0.3) (layers "F.Cu" "B.Cu") (free yes) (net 4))
 (via (at 108.25 102.9) (size 0.6) (drill 0.3) (layers "F.Cu" "B.Cu") (free yes) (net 4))
 (via (at 103.1 110.6) (size 0.6) (drill 0.3) (layers "F.Cu" "B.Cu") (free yes) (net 4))
 (via (at 103 107.8) (size 0.6) (drill 0.3) (layers "F.Cu" "B.Cu") (free yes) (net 4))
 (via (at 104.4 103.4) (size 0.6) (drill 0.3) (layers "F.Cu" "B.Cu") (free yes) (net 4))
 (via (at 121.75 102.9) (size 0.6) (drill 0.3) (layers "F.Cu" "B.Cu") (free yes) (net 4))
 (via (at 102.4 106) (size 0.6) (drill 0.3) (layers "F.Cu" "B.Cu") (free yes) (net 4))
 (segment (start 103.6 102.6) (end 104 102.2) (width 0.2) (layer "F.Cu") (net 5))
 (segment (start 119.925 100.7) (end 120 100.775) (width 0.2) (layer "F.Cu") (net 5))
 (segment (start 103.6 109.2) (end 103.6 102.6) (width 0.2) (layer "F.Cu") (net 5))
 (segment (start 118.6 100.7) (end 119.925 100.7) (width 0.2) (layer "F.Cu") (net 5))
 (segment (start 120 100.775) (end 120 105.025) (width 0.2) (layer "F.Cu") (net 5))
 (via (at 104 102.2) (size 0.6) (drill 0.3) (layers "F.Cu" "B.Cu") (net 5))
 (via (at 118.6 100.7) (size 0.6) (drill 0.3) (layers "F.Cu" "B.Cu") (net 5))
 (segment (start 105.5 100.7) (end 118.6 100.7) (width 0.2) (layer "B.Cu") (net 5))
 (segment (start 104 102.2) (end 105.5 100.7) (width 0.2) (layer "B.Cu") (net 5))
 (segment (start 106.425 100.7) (end 106.5 100.775) (width 0.2) (layer "F.Cu") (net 3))
 (segment (start 102.6 109.2) (end 102.6 108.574602) (width 0.2) (layer "F.Cu") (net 3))
 (segment (start 106.5 100.775) (end 106.5 105.025) (width 0.2) (layer "F.Cu") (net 3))
 (segment (start 102.6 108.574602) (end 102.3322 108.306802) (width 0.2) (layer "F.Cu") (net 3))
 (via (at 106.5 102.9) (size 0.6) (drill 0.3) (layers "F.Cu" "B.Cu") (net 3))
 (via (at 102.3322 108.306802) (size 0.6) (drill 0.3) (layers "F.Cu" "B.Cu") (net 3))
 (segment (start 102.3322 107.0678) (end 106.5 102.9) (width 0.2) (layer "B.Cu") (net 3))
 (segment (start 102.3322 108.306802) (end 102.3322 107.0678) (width 0.2) (layer "B.Cu") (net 3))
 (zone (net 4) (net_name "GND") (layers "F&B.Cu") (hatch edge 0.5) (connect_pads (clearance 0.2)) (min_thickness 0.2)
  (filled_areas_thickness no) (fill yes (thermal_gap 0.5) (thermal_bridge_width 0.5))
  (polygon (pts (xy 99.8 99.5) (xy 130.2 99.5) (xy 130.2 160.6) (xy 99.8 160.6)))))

